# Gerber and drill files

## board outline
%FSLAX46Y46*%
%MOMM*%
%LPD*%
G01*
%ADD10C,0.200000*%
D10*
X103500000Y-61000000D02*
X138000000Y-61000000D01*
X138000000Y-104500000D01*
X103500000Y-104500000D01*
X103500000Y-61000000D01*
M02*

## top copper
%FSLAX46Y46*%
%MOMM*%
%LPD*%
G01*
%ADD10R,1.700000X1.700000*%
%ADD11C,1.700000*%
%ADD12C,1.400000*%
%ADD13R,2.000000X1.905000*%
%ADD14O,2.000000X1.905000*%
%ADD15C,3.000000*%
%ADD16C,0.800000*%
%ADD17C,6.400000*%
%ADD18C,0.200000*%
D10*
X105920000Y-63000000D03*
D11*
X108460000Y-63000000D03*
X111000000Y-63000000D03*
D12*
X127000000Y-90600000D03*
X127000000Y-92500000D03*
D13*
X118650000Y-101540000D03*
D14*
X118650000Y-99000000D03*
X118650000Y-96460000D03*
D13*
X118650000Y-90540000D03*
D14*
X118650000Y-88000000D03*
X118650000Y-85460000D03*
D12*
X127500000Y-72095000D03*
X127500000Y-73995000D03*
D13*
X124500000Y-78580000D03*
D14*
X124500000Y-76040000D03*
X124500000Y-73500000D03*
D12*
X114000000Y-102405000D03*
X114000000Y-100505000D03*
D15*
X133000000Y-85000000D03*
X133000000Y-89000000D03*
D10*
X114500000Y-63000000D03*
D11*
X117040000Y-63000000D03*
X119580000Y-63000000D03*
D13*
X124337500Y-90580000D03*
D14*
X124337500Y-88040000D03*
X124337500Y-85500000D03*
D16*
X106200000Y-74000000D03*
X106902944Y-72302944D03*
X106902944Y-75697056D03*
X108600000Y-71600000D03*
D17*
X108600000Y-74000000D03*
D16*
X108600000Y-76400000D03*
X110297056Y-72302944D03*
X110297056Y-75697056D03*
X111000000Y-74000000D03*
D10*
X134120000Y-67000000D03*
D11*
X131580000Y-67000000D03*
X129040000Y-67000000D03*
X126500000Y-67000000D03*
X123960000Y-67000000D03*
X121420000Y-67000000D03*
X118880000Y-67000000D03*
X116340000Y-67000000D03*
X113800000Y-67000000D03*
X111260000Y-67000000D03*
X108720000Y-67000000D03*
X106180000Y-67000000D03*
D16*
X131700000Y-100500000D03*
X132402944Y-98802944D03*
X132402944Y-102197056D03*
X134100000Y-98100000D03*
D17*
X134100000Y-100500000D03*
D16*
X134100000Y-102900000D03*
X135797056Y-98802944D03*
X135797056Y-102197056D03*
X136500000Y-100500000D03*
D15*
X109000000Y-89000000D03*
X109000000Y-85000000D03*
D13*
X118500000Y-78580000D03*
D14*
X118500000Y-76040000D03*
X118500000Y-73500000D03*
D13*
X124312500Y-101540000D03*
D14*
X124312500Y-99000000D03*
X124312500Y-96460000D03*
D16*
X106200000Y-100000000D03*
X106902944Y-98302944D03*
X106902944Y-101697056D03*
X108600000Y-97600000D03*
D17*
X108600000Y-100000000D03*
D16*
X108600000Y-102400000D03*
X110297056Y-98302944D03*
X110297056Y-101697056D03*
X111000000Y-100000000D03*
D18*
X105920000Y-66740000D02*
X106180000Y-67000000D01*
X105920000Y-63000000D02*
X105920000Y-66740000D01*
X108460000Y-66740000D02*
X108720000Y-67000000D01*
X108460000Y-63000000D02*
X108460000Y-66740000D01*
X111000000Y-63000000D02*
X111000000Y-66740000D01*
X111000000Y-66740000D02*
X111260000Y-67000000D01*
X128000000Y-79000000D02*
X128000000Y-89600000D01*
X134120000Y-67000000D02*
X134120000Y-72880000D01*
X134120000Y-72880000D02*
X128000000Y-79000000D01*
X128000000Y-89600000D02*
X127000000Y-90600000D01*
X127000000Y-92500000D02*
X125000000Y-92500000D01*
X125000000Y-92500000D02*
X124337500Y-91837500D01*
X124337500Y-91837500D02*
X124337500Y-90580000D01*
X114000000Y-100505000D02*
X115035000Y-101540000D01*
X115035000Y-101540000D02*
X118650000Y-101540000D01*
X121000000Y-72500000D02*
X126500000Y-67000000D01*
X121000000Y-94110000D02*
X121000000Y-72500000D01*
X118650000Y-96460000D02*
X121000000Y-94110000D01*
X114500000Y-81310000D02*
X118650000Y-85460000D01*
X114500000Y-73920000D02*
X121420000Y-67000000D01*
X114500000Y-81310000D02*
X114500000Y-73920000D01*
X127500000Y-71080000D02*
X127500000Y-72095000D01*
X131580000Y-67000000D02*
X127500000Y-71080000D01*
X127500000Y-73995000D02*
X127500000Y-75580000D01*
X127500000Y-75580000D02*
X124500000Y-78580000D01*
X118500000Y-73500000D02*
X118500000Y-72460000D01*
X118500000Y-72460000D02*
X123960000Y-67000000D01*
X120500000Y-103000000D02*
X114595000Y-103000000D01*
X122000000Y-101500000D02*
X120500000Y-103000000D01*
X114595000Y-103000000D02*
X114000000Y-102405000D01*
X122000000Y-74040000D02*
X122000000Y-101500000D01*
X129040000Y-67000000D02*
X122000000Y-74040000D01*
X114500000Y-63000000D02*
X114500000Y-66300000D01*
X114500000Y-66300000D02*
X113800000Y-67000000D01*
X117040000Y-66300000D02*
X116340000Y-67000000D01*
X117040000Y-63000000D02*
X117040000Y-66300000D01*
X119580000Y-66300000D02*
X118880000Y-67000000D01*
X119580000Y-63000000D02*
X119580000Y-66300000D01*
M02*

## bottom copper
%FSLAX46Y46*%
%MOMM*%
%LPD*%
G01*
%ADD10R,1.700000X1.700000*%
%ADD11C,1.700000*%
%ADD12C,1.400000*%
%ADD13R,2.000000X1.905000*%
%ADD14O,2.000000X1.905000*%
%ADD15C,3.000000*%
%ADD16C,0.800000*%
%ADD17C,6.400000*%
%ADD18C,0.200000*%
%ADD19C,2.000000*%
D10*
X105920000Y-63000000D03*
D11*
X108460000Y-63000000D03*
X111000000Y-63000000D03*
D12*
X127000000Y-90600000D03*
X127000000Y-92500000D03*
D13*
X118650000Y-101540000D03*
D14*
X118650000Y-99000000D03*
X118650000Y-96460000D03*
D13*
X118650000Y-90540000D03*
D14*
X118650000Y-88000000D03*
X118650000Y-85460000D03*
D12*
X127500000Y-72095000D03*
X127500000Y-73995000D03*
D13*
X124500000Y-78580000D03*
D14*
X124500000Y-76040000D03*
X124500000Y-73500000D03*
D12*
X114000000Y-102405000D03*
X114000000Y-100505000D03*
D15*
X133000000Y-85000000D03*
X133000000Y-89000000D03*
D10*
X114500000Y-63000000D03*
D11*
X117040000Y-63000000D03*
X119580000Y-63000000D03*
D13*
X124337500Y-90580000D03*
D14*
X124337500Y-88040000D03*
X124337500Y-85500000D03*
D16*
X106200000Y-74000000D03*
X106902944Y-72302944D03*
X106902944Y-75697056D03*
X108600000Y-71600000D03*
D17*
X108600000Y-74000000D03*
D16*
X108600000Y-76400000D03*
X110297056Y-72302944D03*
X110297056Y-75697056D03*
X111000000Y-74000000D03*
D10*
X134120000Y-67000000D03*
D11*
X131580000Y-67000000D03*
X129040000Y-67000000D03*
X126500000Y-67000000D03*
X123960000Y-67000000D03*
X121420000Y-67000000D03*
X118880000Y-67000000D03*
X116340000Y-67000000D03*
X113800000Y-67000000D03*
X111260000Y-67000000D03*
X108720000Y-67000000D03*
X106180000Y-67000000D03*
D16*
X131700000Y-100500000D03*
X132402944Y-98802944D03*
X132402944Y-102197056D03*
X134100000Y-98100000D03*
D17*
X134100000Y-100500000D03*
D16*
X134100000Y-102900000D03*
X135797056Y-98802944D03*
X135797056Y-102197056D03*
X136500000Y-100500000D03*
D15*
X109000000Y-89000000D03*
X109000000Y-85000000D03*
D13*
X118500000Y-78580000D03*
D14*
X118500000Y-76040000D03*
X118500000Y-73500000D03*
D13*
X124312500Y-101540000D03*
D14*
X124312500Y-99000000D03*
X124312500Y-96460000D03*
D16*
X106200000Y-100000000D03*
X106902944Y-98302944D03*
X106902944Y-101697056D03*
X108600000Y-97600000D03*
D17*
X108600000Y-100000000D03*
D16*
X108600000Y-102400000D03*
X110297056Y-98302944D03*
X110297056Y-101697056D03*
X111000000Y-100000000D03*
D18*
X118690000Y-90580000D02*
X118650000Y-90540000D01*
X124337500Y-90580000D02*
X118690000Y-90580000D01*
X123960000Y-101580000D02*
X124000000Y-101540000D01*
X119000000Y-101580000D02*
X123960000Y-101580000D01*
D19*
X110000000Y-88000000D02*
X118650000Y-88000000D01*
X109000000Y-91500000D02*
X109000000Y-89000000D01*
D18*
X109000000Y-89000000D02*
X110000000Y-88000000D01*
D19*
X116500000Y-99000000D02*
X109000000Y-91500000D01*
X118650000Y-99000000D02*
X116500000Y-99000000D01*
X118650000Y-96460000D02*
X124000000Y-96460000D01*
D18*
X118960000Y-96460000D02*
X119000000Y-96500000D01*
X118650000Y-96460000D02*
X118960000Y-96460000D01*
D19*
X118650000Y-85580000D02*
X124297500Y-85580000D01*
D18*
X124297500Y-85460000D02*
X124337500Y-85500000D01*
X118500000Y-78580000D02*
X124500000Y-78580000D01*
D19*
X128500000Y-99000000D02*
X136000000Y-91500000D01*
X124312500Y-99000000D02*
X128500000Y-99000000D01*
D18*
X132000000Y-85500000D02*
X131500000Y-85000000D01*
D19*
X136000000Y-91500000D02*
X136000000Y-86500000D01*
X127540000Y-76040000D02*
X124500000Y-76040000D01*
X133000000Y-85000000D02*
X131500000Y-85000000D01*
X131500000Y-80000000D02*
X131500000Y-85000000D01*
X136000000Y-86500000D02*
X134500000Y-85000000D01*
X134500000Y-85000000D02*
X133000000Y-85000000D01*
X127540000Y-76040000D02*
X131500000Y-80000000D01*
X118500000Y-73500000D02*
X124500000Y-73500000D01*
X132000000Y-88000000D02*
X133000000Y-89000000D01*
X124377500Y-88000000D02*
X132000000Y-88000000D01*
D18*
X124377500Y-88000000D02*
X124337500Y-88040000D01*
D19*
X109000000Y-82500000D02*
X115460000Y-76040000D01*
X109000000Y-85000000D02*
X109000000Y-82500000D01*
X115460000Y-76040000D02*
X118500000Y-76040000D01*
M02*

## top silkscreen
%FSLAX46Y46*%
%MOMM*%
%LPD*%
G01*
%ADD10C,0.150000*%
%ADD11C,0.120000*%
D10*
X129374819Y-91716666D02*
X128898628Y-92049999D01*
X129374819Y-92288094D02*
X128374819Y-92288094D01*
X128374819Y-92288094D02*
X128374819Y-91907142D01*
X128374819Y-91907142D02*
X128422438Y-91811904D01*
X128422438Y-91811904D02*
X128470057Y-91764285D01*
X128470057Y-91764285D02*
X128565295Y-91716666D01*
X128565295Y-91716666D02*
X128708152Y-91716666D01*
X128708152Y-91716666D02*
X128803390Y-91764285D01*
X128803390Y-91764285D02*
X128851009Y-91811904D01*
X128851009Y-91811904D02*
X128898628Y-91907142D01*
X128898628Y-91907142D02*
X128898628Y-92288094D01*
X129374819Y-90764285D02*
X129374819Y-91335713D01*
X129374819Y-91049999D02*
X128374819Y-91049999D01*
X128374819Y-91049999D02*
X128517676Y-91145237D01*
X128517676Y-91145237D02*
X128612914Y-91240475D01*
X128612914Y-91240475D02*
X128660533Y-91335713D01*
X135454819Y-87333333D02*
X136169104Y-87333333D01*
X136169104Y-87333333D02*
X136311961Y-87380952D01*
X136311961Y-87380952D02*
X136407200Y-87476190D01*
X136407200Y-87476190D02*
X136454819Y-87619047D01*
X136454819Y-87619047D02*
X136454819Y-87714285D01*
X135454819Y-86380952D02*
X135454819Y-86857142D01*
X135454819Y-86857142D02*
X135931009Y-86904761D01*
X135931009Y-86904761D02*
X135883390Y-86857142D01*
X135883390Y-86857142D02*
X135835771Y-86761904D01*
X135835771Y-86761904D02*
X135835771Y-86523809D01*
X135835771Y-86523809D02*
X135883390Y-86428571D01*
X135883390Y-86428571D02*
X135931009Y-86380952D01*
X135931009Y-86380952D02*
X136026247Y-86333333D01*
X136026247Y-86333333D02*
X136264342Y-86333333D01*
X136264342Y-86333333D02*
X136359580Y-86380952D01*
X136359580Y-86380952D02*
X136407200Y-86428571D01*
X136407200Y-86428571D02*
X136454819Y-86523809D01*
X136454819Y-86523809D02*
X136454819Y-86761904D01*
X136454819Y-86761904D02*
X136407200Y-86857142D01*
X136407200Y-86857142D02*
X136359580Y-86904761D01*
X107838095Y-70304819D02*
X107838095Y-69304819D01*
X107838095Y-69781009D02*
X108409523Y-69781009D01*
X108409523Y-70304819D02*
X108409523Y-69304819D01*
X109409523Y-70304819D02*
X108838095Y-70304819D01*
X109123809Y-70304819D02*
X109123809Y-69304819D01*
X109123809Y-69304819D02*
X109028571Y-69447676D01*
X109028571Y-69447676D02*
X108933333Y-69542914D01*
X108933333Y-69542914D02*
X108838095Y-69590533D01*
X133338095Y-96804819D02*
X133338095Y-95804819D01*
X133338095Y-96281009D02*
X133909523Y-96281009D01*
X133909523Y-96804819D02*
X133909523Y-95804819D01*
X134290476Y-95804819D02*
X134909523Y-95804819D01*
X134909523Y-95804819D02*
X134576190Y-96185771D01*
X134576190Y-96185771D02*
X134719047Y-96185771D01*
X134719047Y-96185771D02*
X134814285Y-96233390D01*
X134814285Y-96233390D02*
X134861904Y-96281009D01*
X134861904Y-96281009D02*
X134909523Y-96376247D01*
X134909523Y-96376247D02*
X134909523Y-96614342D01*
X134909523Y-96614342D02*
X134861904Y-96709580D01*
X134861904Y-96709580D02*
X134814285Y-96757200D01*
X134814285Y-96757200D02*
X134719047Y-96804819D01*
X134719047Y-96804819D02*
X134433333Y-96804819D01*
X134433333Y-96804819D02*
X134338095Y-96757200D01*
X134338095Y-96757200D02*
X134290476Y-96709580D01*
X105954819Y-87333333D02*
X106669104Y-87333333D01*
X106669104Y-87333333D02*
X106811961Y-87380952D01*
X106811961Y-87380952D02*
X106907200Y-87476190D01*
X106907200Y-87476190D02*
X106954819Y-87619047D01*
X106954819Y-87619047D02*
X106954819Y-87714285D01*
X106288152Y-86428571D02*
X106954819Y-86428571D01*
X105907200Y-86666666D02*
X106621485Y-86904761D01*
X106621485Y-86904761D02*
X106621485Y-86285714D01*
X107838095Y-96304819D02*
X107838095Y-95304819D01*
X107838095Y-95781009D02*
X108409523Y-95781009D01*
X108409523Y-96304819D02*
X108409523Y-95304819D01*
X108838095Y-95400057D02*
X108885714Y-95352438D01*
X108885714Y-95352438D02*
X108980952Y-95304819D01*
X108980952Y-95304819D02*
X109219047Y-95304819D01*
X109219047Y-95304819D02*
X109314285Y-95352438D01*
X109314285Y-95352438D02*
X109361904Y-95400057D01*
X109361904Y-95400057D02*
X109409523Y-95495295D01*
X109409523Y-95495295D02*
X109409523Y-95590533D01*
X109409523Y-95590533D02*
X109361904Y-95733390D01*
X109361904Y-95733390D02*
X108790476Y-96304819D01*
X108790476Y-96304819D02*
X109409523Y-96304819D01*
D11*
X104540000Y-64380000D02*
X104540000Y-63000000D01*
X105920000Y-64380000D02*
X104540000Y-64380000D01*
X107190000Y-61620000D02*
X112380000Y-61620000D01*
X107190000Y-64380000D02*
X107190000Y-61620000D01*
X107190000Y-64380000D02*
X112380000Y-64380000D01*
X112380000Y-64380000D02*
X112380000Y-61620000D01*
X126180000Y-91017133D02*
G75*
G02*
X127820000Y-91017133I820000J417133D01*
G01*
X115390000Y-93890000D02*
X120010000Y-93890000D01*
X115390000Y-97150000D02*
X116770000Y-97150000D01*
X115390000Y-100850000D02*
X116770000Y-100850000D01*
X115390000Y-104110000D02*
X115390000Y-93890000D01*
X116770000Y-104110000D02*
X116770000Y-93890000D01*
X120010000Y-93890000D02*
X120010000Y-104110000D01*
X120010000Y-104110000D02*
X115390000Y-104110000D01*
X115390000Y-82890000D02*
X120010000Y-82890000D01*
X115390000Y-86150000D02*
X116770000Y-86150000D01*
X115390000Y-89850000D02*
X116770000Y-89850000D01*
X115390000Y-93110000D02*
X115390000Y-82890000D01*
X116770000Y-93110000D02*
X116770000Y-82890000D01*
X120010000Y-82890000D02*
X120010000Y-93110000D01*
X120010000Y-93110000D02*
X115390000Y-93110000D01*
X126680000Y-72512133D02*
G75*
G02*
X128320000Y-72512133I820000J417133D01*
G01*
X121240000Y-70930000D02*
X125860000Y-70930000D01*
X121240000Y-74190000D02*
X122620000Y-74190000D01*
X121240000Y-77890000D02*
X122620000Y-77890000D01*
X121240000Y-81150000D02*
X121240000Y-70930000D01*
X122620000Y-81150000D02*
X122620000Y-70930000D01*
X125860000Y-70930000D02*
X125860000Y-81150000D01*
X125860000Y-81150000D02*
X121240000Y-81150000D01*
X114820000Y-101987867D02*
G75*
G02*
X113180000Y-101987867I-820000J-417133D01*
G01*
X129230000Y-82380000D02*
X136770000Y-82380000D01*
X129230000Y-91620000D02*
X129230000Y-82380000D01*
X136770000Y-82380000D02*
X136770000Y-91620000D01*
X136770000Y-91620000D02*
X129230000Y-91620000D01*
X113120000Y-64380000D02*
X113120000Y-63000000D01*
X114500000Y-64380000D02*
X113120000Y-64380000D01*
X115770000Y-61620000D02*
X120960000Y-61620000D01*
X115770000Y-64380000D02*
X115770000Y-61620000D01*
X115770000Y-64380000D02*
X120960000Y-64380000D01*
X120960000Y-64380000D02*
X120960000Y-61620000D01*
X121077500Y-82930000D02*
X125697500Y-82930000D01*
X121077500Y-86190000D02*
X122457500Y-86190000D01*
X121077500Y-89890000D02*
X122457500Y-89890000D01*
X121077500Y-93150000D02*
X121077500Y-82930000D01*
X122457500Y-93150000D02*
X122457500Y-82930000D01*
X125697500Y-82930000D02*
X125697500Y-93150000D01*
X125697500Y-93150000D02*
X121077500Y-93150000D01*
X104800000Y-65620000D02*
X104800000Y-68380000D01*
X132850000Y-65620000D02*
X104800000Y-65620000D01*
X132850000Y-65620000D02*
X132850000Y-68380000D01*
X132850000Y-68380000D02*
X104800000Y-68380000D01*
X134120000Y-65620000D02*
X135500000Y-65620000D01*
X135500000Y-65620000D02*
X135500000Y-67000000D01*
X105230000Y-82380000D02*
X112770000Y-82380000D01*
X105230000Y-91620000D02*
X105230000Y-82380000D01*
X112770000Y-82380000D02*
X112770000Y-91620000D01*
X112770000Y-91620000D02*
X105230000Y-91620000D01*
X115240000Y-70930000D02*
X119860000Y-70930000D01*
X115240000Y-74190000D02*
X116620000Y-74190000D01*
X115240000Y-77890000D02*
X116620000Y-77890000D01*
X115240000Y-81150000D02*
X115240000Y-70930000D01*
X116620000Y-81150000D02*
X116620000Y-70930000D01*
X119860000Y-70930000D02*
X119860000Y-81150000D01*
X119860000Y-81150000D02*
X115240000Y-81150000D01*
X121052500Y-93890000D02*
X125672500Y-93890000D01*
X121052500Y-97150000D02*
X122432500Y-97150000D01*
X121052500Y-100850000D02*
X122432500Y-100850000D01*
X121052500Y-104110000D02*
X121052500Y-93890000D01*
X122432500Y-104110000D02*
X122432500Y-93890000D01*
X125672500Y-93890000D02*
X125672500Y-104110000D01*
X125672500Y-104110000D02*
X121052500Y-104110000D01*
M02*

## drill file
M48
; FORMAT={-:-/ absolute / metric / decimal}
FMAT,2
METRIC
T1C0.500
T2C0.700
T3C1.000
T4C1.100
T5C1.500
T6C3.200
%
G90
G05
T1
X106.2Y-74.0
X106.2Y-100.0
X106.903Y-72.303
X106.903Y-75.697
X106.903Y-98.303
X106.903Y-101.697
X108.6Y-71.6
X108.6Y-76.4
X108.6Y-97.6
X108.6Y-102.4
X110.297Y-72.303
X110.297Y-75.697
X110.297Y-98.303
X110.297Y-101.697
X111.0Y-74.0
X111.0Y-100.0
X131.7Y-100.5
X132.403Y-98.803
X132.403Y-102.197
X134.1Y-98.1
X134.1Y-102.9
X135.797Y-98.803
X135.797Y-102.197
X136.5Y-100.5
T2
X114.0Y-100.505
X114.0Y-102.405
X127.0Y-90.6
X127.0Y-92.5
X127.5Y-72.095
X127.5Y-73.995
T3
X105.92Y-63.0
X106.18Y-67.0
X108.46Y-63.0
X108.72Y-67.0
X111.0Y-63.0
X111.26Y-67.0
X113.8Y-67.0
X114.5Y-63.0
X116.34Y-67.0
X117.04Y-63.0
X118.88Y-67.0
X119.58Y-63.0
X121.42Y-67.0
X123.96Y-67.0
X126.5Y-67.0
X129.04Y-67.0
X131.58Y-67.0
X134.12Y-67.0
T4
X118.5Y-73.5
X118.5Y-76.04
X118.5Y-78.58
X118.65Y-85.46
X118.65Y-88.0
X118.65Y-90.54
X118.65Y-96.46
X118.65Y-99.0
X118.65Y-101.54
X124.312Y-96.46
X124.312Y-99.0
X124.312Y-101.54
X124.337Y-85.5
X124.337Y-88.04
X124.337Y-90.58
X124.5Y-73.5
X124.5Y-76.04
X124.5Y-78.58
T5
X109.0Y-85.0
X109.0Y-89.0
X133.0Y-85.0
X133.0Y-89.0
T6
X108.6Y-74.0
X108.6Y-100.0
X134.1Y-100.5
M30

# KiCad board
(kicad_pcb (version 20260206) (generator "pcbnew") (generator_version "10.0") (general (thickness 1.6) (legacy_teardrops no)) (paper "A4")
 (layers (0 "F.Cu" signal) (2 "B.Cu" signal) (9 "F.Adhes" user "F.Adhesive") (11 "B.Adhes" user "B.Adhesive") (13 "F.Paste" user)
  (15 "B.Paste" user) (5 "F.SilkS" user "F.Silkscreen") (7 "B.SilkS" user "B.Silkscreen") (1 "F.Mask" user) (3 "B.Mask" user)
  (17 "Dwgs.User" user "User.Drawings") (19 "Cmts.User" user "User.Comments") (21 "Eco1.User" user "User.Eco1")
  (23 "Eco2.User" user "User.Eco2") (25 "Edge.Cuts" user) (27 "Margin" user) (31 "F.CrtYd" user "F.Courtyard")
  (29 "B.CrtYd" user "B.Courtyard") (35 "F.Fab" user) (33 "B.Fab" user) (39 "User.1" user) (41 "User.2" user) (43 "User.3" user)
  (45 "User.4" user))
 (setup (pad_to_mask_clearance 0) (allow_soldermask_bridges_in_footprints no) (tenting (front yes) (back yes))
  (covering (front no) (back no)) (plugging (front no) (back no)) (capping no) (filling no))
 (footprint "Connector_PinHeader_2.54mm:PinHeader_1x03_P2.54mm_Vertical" (layer "F.Cu") (at 105.92 63 90)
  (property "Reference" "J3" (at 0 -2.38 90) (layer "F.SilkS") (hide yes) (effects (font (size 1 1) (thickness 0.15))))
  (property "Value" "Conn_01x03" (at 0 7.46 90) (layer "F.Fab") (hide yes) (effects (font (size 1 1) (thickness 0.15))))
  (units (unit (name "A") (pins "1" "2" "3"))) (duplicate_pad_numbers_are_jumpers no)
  (fp_line (start -1.38 -1.38) (end 0 -1.38) (stroke (width 0.12) (type solid)) (layer "F.SilkS"))
  (fp_line (start -1.38 0) (end -1.38 -1.38) (stroke (width 0.12) (type solid)) (layer "F.SilkS"))
  (fp_line (start 1.38 1.27) (end 1.38 6.46) (stroke (width 0.12) (type solid)) (layer "F.SilkS"))
  (fp_line (start -1.38 1.27) (end 1.38 1.27) (stroke (width 0.12) (type solid)) (layer "F.SilkS"))
  (fp_line (start -1.38 1.27) (end -1.38 6.46) (stroke (width 0.12) (type solid)) (layer "F.SilkS"))
  (fp_line (start -1.38 6.46) (end 1.38 6.46) (stroke (width 0.12) (type solid)) (layer "F.SilkS"))
  (pad "1" thru_hole rect (at 0 0 90) (size 1.7 1.7) (drill 1) (layers "*.Cu" "*.Mask") (remove_unused_layers no) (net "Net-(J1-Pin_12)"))
  (pad "2" thru_hole circle (at 0 2.54 90) (size 1.7 1.7) (drill 1) (layers "*.Cu" "*.Mask") (remove_unused_layers no)
   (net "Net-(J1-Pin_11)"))
  (pad "3" thru_hole circle (at 0 5.08 90) (size 1.7 1.7) (drill 1) (layers "*.Cu" "*.Mask") (remove_unused_layers no)
   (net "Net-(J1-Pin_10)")))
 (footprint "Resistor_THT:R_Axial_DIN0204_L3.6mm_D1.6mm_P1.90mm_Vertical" (layer "F.Cu") (at 127 90.6 -90)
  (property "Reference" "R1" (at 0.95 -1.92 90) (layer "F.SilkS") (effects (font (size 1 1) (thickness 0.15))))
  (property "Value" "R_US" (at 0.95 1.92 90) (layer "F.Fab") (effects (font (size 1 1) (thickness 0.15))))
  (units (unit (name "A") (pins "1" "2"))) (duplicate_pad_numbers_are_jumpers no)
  (fp_arc (start 0.417133 0.82) (mid -0.92 0) (end 0.417133 -0.82) (stroke (width 0.12) (type solid)) (layer "F.SilkS"))
  (pad "1" thru_hole circle (at 0 0 270) (size 1.4 1.4) (drill 0.7) (layers "*.Cu" "*.Mask") (remove_unused_layers no)
   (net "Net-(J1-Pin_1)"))
  (pad "2" thru_hole circle (at 1.9 0 270) (size 1.4 1.4) (drill 0.7) (layers "*.Cu" "*.Mask") (remove_unused_layers no) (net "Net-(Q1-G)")))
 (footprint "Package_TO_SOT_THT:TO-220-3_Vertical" (layer "F.Cu") (at 118.65 101.54 90)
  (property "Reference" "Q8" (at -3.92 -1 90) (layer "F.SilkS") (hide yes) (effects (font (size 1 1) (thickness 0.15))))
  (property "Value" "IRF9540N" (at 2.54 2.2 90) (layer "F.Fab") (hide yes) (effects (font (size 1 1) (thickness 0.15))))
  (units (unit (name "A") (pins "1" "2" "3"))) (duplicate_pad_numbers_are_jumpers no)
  (fp_line (start 7.65 -3.26) (end 7.65 1.36) (stroke (width 0.12) (type solid)) (layer "F.SilkS"))
  (fp_line (start 4.39 -3.26) (end 4.39 -1.88) (stroke (width 0.12) (type solid)) (layer "F.SilkS"))
  (fp_line (start 0.69 -3.26) (end 0.69 -1.88) (stroke (width 0.12) (type solid)) (layer "F.SilkS"))
  (fp_line (start -2.57 -3.26) (end 7.65 -3.26) (stroke (width 0.12) (type solid)) (layer "F.SilkS"))
  (fp_line (start -2.57 -1.88) (end 7.65 -1.88) (stroke (width 0.12) (type solid)) (layer "F.SilkS"))
  (fp_line (start 7.65 1.36) (end -2.57 1.36) (stroke (width 0.12) (type solid)) (layer "F.SilkS"))
  (fp_line (start -2.57 1.36) (end -2.57 -3.26) (stroke (width 0.12) (type solid)) (layer "F.SilkS"))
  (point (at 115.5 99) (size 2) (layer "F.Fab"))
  (pad "1" thru_hole rect (at 0 0 90) (size 1.905 2) (drill 1.1) (layers "*.Cu" "*.Mask") (remove_unused_layers no) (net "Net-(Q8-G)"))
  (pad "2" thru_hole oval (at 2.54 0 90) (size 1.905 2) (drill 1.1) (layers "*.Cu" "*.Mask") (remove_unused_layers no) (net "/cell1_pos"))
  (pad "3" thru_hole oval (at 5.08 0 90) (size 1.905 2) (drill 1.1) (layers "*.Cu" "*.Mask") (remove_unused_layers no) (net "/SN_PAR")))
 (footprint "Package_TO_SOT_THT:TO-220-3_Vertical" (layer "F.Cu") (at 118.65 90.54 90)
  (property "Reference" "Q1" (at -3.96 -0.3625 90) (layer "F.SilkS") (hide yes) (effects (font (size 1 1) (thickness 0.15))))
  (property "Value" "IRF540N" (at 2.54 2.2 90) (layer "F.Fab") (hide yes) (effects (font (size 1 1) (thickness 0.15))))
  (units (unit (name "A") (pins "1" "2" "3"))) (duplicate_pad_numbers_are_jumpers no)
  (fp_line (start 7.65 -3.26) (end 7.65 1.36) (stroke (width 0.12) (type solid)) (layer "F.SilkS"))
  (fp_line (start 4.39 -3.26) (end 4.39 -1.88) (stroke (width 0.12) (type solid)) (layer "F.SilkS"))
  (fp_line (start 0.69 -3.26) (end 0.69 -1.88) (stroke (width 0.12) (type solid)) (layer "F.SilkS"))
  (fp_line (start -2.57 -3.26) (end 7.65 -3.26) (stroke (width 0.12) (type solid)) (layer "F.SilkS"))
  (fp_line (start -2.57 -1.88) (end 7.65 -1.88) (stroke (width 0.12) (type solid)) (layer "F.SilkS"))
  (fp_line (start 7.65 1.36) (end -2.57 1.36) (stroke (width 0.12) (type solid)) (layer "F.SilkS"))
  (fp_line (start -2.57 1.36) (end -2.57 -3.26) (stroke (width 0.12) (type solid)) (layer "F.SilkS"))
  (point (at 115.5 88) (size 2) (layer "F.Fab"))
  (pad "1" thru_hole rect (at 0 0 90) (size 1.905 2) (drill 1.1) (layers "*.Cu" "*.Mask") (remove_unused_layers no) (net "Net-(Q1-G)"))
  (pad "2" thru_hole oval (at 2.54 0 90) (size 1.905 2) (drill 1.1) (layers "*.Cu" "*.Mask") (remove_unused_layers no) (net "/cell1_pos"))
  (pad "3" thru_hole oval (at 5.08 0 90) (size 1.905 2) (drill 1.1) (layers "*.Cu" "*.Mask") (remove_unused_layers no) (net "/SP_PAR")))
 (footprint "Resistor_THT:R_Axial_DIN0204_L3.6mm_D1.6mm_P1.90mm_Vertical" (layer "F.Cu") (at 127.5 72.095 -90)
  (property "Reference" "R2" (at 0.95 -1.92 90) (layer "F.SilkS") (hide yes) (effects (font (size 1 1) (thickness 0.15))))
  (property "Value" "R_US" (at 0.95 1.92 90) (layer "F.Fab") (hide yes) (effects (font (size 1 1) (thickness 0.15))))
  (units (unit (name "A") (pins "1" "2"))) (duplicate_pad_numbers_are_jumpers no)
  (fp_arc (start 0.417133 0.82) (mid -0.92 0) (end 0.417133 -0.82) (stroke (width 0.12) (type solid)) (layer "F.SilkS"))
  (pad "1" thru_hole circle (at 0 0 270) (size 1.4 1.4) (drill 0.7) (layers "*.Cu" "*.Mask") (remove_unused_layers no)
   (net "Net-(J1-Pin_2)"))
  (pad "2" thru_hole circle (at 1.9 0 270) (size 1.4 1.4) (drill 0.7) (layers "*.Cu" "*.Mask") (remove_unused_layers no) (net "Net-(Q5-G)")))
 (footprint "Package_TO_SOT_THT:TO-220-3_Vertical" (layer "F.Cu") (at 124.5 78.58 90)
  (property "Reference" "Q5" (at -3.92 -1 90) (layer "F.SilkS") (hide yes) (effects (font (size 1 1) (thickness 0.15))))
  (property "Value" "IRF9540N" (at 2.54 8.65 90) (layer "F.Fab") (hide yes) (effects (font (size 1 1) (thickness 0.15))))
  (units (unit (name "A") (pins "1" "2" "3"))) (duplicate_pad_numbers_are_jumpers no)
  (fp_line (start 7.65 -3.26) (end 7.65 1.36) (stroke (width 0.12) (type solid)) (layer "F.SilkS"))
  (fp_line (start 4.39 -3.26) (end 4.39 -1.88) (stroke (width 0.12) (type solid)) (layer "F.SilkS"))
  (fp_line (start 0.69 -3.26) (end 0.69 -1.88) (stroke (width 0.12) (type solid)) (layer "F.SilkS"))
  (fp_line (start -2.57 -3.26) (end 7.65 -3.26) (stroke (width 0.12) (type solid)) (layer "F.SilkS"))
  (fp_line (start -2.57 -1.88) (end 7.65 -1.88) (stroke (width 0.12) (type solid)) (layer "F.SilkS"))
  (fp_line (start 7.65 1.36) (end -2.57 1.36) (stroke (width 0.12) (type solid)) (layer "F.SilkS"))
  (fp_line (start -2.57 1.36) (end -2.57 -3.26) (stroke (width 0.12) (type solid)) (layer "F.SilkS"))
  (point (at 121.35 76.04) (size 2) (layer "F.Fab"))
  (pad "1" thru_hole rect (at 0 0 90) (size 1.905 2) (drill 1.1) (layers "*.Cu" "*.Mask") (remove_unused_layers no) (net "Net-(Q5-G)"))
  (pad "2" thru_hole oval (at 2.54 0 90) (size 1.905 2) (drill 1.1) (layers "*.Cu" "*.Mask") (remove_unused_layers no) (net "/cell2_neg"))
  (pad "3" thru_hole oval (at 5.08 0 90) (size 1.905 2) (drill 1.1) (layers "*.Cu" "*.Mask") (remove_unused_layers no) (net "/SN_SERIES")))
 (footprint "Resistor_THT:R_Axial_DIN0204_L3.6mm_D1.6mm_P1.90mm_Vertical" (layer "F.Cu") (at 114 102.405 90)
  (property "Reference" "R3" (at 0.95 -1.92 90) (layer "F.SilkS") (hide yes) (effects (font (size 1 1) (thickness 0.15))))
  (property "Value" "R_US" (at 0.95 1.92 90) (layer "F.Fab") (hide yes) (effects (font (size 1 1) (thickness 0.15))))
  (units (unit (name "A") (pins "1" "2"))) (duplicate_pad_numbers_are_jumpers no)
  (fp_arc (start 0.417133 0.82) (mid -0.92 0) (end 0.417133 -0.82) (stroke (width 0.12) (type solid)) (layer "F.SilkS"))
  (pad "1" thru_hole circle (at 0 0 90) (size 1.4 1.4) (drill 0.7) (layers "*.Cu" "*.Mask") (remove_unused_layers no) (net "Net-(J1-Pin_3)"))
  (pad "2" thru_hole circle (at 1.9 0 90) (size 1.4 1.4) (drill 0.7) (layers "*.Cu" "*.Mask") (remove_unused_layers no) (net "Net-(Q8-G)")))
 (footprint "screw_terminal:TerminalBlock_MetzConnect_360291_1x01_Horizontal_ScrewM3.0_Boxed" (layer "F.Cu") (at 133 85 -90)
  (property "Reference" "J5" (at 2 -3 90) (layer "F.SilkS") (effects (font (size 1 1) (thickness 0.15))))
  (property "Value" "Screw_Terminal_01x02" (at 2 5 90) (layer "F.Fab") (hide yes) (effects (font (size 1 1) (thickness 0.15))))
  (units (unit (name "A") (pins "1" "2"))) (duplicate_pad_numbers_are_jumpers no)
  (fp_line (start -2.62 3.77) (end -2.62 -3.77) (stroke (width 0.12) (type solid)) (layer "F.SilkS"))
  (fp_line (start 6.62 3.77) (end -2.62 3.77) (stroke (width 0.12) (type solid)) (layer "F.SilkS"))
  (fp_line (start -2.62 -3.77) (end 6.62 -3.77) (stroke (width 0.12) (type solid)) (layer "F.SilkS"))
  (fp_line (start 6.62 -3.77) (end 6.62 3.77) (stroke (width 0.12) (type solid)) (layer "F.SilkS"))
  (pad "1" thru_hole circle (at 0 0 270) (size 3 3) (drill 1.5) (layers "*.Cu" "*.Mask") (remove_unused_layers no) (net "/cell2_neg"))
  (pad "2" thru_hole circle (at 4 0 270) (size 3 3) (drill 1.5) (layers "*.Cu" "*.Mask") (remove_unused_layers no) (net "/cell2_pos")))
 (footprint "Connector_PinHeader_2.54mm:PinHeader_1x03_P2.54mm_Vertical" (layer "F.Cu") (at 114.5 63 90)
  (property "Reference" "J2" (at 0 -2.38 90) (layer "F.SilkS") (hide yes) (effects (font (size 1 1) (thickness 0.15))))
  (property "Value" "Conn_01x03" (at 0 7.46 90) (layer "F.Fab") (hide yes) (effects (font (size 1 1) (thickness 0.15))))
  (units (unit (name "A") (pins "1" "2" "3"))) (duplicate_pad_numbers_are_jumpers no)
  (fp_line (start -1.38 -1.38) (end 0 -1.38) (stroke (width 0.12) (type solid)) (layer "F.SilkS"))
  (fp_line (start -1.38 0) (end -1.38 -1.38) (stroke (width 0.12) (type solid)) (layer "F.SilkS"))
  (fp_line (start 1.38 1.27) (end 1.38 6.46) (stroke (width 0.12) (type solid)) (layer "F.SilkS"))
  (fp_line (start -1.38 1.27) (end 1.38 1.27) (stroke (width 0.12) (type solid)) (layer "F.SilkS"))
  (fp_line (start -1.38 1.27) (end -1.38 6.46) (stroke (width 0.12) (type solid)) (layer "F.SilkS"))
  (fp_line (start -1.38 6.46) (end 1.38 6.46) (stroke (width 0.12) (type solid)) (layer "F.SilkS"))
  (pad "1" thru_hole rect (at 0 0 90) (size 1.7 1.7) (drill 1) (layers "*.Cu" "*.Mask") (remove_unused_layers no) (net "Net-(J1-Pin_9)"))
  (pad "2" thru_hole circle (at 0 2.54 90) (size 1.7 1.7) (drill 1) (layers "*.Cu" "*.Mask") (remove_unused_layers no)
   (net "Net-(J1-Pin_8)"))
  (pad "3" thru_hole circle (at 0 5.08 90) (size 1.7 1.7) (drill 1) (layers "*.Cu" "*.Mask") (remove_unused_layers no)
   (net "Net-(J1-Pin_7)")))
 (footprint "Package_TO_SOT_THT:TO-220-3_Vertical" (layer "F.Cu") (at 124.3375 90.58 90)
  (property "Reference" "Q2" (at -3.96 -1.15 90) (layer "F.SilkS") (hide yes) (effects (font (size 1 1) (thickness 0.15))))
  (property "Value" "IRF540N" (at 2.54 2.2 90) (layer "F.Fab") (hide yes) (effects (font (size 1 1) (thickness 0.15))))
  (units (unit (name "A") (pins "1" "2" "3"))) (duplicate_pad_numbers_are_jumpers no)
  (fp_line (start 7.65 -3.26) (end 7.65 1.36) (stroke (width 0.12) (type solid)) (layer "F.SilkS"))
  (fp_line (start 4.39 -3.26) (end 4.39 -1.88) (stroke (width 0.12) (type solid)) (layer "F.SilkS"))
  (fp_line (start 0.69 -3.26) (end 0.69 -1.88) (stroke (width 0.12) (type solid)) (layer "F.SilkS"))
  (fp_line (start -2.57 -3.26) (end 7.65 -3.26) (stroke (width 0.12) (type solid)) (layer "F.SilkS"))
  (fp_line (start -2.57 -1.88) (end 7.65 -1.88) (stroke (width 0.12) (type solid)) (layer "F.SilkS"))
  (fp_line (start 7.65 1.36) (end -2.57 1.36) (stroke (width 0.12) (type solid)) (layer "F.SilkS"))
  (fp_line (start -2.57 1.36) (end -2.57 -3.26) (stroke (width 0.12) (type solid)) (layer "F.SilkS"))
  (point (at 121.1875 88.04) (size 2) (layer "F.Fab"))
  (pad "1" thru_hole rect (at 0 0 90) (size 1.905 2) (drill 1.1) (layers "*.Cu" "*.Mask") (remove_unused_layers no) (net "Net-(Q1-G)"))
  (pad "2" thru_hole oval (at 2.54 0 90) (size 1.905 2) (drill 1.1) (layers "*.Cu" "*.Mask") (remove_unused_layers no) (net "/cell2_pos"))
  (pad "3" thru_hole oval (at 5.08 0 90) (size 1.905 2) (drill 1.1) (layers "*.Cu" "*.Mask") (remove_unused_layers no) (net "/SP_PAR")))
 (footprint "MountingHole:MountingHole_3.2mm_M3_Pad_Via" (layer "F.Cu") (at 108.6 74)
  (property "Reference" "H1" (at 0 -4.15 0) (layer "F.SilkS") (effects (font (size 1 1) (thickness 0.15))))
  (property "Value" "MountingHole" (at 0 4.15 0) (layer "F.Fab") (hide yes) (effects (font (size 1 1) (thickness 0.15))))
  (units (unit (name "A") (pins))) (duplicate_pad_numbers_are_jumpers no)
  (pad "1" thru_hole circle (at -2.4 0) (size 0.8 0.8) (drill 0.5) (layers "*.Cu" "*.Mask") (remove_unused_layers no) (zone_connect 2))
  (pad "1" thru_hole circle (at -1.697056 -1.697056) (size 0.8 0.8) (drill 0.5) (layers "*.Cu" "*.Mask") (remove_unused_layers no)
   (zone_connect 2))
  (pad "1" thru_hole circle (at -1.697056 1.697056) (size 0.8 0.8) (drill 0.5) (layers "*.Cu" "*.Mask") (remove_unused_layers no)
   (zone_connect 2))
  (pad "1" thru_hole circle (at 0 -2.4) (size 0.8 0.8) (drill 0.5) (layers "*.Cu" "*.Mask") (remove_unused_layers no) (zone_connect 2))
  (pad "1" thru_hole circle (at 0 0) (size 6.4 6.4) (drill 3.2) (layers "*.Cu" "*.Mask") (remove_unused_layers no) (zone_connect 2))
  (pad "1" thru_hole circle (at 0 2.4) (size 0.8 0.8) (drill 0.5) (layers "*.Cu" "*.Mask") (remove_unused_layers no) (zone_connect 2))
  (pad "1" thru_hole circle (at 1.697056 -1.697056) (size 0.8 0.8) (drill 0.5) (layers "*.Cu" "*.Mask") (remove_unused_layers no)
   (zone_connect 2))
  (pad "1" thru_hole circle (at 1.697056 1.697056) (size 0.8 0.8) (drill 0.5) (layers "*.Cu" "*.Mask") (remove_unused_layers no)
   (zone_connect 2))
  (pad "1" thru_hole circle (at 2.4 0) (size 0.8 0.8) (drill 0.5) (layers "*.Cu" "*.Mask") (remove_unused_layers no) (zone_connect 2)))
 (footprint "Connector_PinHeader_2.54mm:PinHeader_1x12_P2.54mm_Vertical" (layer "F.Cu") (at 134.12 67 -90)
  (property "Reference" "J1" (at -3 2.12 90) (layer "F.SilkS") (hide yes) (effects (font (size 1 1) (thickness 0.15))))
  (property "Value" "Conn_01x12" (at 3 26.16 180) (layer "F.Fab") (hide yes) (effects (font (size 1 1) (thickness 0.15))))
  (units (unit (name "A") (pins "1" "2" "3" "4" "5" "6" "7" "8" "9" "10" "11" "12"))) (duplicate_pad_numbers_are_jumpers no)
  (fp_line (start -1.38 29.32) (end 1.38 29.32) (stroke (width 0.12) (type solid)) (layer "F.SilkS"))
  (fp_line (start -1.38 1.27) (end -1.38 29.32) (stroke (width 0.12) (type solid)) (layer "F.SilkS"))
  (fp_line (start -1.38 1.27) (end 1.38 1.27) (stroke (width 0.12) (type solid)) (layer "F.SilkS"))
  (fp_line (start 1.38 1.27) (end 1.38 29.32) (stroke (width 0.12) (type solid)) (layer "F.SilkS"))
  (fp_line (start -1.38 0) (end -1.38 -1.38) (stroke (width 0.12) (type solid)) (layer "F.SilkS"))
  (fp_line (start -1.38 -1.38) (end 0 -1.38) (stroke (width 0.12) (type solid)) (layer "F.SilkS"))
  (pad "1" thru_hole rect (at 0 0 270) (size 1.7 1.7) (drill 1) (layers "*.Cu" "*.Mask") (remove_unused_layers no) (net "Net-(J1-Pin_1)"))
  (pad "2" thru_hole circle (at 0 2.54 270) (size 1.7 1.7) (drill 1) (layers "*.Cu" "*.Mask") (remove_unused_layers no)
   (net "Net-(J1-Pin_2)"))
  (pad "3" thru_hole circle (at 0 5.08 270) (size 1.7 1.7) (drill 1) (layers "*.Cu" "*.Mask") (remove_unused_layers no)
   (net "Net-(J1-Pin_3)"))
  (pad "4" thru_hole circle (at 0 7.62 270) (size 1.7 1.7) (drill 1) (layers "*.Cu" "*.Mask") (remove_unused_layers no) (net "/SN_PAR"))
  (pad "5" thru_hole circle (at 0 10.16 270) (size 1.7 1.7) (drill 1) (layers "*.Cu" "*.Mask") (remove_unused_layers no) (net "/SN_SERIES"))
  (pad "6" thru_hole circle (at 0 12.7 270) (size 1.7 1.7) (drill 1) (layers "*.Cu" "*.Mask") (remove_unused_layers no) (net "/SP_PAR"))
  (pad "7" thru_hole circle (at 0 15.24 270) (size 1.7 1.7) (drill 1) (layers "*.Cu" "*.Mask") (remove_unused_layers no)
   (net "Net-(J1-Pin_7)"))
  (pad "8" thru_hole circle (at 0 17.78 270) (size 1.7 1.7) (drill 1) (layers "*.Cu" "*.Mask") (remove_unused_layers no)
   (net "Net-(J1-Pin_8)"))
  (pad "9" thru_hole circle (at 0 20.32 270) (size 1.7 1.7) (drill 1) (layers "*.Cu" "*.Mask") (remove_unused_layers no)
   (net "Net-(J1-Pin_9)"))
  (pad "10" thru_hole circle (at 0 22.86 270) (size 1.7 1.7) (drill 1) (layers "*.Cu" "*.Mask") (remove_unused_layers no)
   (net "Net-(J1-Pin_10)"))
  (pad "11" thru_hole circle (at 0 25.4 270) (size 1.7 1.7) (drill 1) (layers "*.Cu" "*.Mask") (remove_unused_layers no)
   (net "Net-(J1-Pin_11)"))
  (pad "12" thru_hole circle (at 0 27.94 270) (size 1.7 1.7) (drill 1) (layers "*.Cu" "*.Mask") (remove_unused_layers no)
   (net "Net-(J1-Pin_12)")))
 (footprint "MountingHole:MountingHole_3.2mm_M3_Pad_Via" (layer "F.Cu") (at 134.1 100.5)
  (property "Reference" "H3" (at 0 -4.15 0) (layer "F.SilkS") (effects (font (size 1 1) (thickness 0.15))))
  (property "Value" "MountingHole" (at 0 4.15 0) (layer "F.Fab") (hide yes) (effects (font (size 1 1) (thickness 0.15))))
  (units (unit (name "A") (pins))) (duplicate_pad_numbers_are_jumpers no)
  (pad "1" thru_hole circle (at -2.4 0) (size 0.8 0.8) (drill 0.5) (layers "*.Cu" "*.Mask") (remove_unused_layers no) (zone_connect 2))
  (pad "1" thru_hole circle (at -1.697056 -1.697056) (size 0.8 0.8) (drill 0.5) (layers "*.Cu" "*.Mask") (remove_unused_layers no)
   (zone_connect 2))
  (pad "1" thru_hole circle (at -1.697056 1.697056) (size 0.8 0.8) (drill 0.5) (layers "*.Cu" "*.Mask") (remove_unused_layers no)
   (zone_connect 2))
  (pad "1" thru_hole circle (at 0 -2.4) (size 0.8 0.8) (drill 0.5) (layers "*.Cu" "*.Mask") (remove_unused_layers no) (zone_connect 2))
  (pad "1" thru_hole circle (at 0 0) (size 6.4 6.4) (drill 3.2) (layers "*.Cu" "*.Mask") (remove_unused_layers no) (zone_connect 2))
  (pad "1" thru_hole circle (at 0 2.4) (size 0.8 0.8) (drill 0.5) (layers "*.Cu" "*.Mask") (remove_unused_layers no) (zone_connect 2))
  (pad "1" thru_hole circle (at 1.697056 -1.697056) (size 0.8 0.8) (drill 0.5) (layers "*.Cu" "*.Mask") (remove_unused_layers no)
   (zone_connect 2))
  (pad "1" thru_hole circle (at 1.697056 1.697056) (size 0.8 0.8) (drill 0.5) (layers "*.Cu" "*.Mask") (remove_unused_layers no)
   (zone_connect 2))
  (pad "1" thru_hole circle (at 2.4 0) (size 0.8 0.8) (drill 0.5) (layers "*.Cu" "*.Mask") (remove_unused_layers no) (zone_connect 2)))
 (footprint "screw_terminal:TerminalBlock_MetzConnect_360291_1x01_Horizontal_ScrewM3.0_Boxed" (layer "F.Cu") (at 109 89 90)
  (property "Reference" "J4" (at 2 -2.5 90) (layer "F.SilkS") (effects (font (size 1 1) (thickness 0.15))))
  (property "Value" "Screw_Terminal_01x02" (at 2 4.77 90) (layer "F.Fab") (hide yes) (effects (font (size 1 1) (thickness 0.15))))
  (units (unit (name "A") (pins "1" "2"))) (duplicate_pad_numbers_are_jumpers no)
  (fp_line (start 6.62 -3.77) (end 6.62 3.77) (stroke (width 0.12) (type solid)) (layer "F.SilkS"))
  (fp_line (start -2.62 -3.77) (end 6.62 -3.77) (stroke (width 0.12) (type solid)) (layer "F.SilkS"))
  (fp_line (start 6.62 3.77) (end -2.62 3.77) (stroke (width 0.12) (type solid)) (layer "F.SilkS"))
  (fp_line (start -2.62 3.77) (end -2.62 -3.77) (stroke (width 0.12) (type solid)) (layer "F.SilkS"))
  (pad "1" thru_hole circle (at 0 0 90) (size 3 3) (drill 1.5) (layers "*.Cu" "*.Mask") (remove_unused_layers no) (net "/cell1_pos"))
  (pad "2" thru_hole circle (at 4 0 90) (size 3 3) (drill 1.5) (layers "*.Cu" "*.Mask") (remove_unused_layers no) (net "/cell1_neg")))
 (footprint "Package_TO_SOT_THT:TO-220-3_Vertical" (layer "F.Cu") (at 118.5 78.58 90)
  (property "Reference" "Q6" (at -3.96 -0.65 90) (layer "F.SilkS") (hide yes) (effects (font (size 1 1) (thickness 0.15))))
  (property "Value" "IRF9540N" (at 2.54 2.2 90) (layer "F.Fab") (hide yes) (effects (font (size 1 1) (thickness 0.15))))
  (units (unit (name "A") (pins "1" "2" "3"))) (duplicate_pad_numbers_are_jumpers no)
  (fp_line (start 7.65 -3.26) (end 7.65 1.36) (stroke (width 0.12) (type solid)) (layer "F.SilkS"))
  (fp_line (start 4.39 -3.26) (end 4.39 -1.88) (stroke (width 0.12) (type solid)) (layer "F.SilkS"))
  (fp_line (start 0.69 -3.26) (end 0.69 -1.88) (stroke (width 0.12) (type solid)) (layer "F.SilkS"))
  (fp_line (start -2.57 -3.26) (end 7.65 -3.26) (stroke (width 0.12) (type solid)) (layer "F.SilkS"))
  (fp_line (start -2.57 -1.88) (end 7.65 -1.88) (stroke (width 0.12) (type solid)) (layer "F.SilkS"))
  (fp_line (start 7.65 1.36) (end -2.57 1.36) (stroke (width 0.12) (type solid)) (layer "F.SilkS"))
  (fp_line (start -2.57 1.36) (end -2.57 -3.26) (stroke (width 0.12) (type solid)) (layer "F.SilkS"))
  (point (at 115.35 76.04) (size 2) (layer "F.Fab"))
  (pad "1" thru_hole rect (at 0 0 90) (size 1.905 2) (drill 1.1) (layers "*.Cu" "*.Mask") (remove_unused_layers no) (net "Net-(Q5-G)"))
  (pad "2" thru_hole oval (at 2.54 0 90) (size 1.905 2) (drill 1.1) (layers "*.Cu" "*.Mask") (remove_unused_layers no) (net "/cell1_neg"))
  (pad "3" thru_hole oval (at 5.08 0 90) (size 1.905 2) (drill 1.1) (layers "*.Cu" "*.Mask") (remove_unused_layers no) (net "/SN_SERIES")))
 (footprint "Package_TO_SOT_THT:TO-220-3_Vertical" (layer "F.Cu") (at 124.3125 101.54 90)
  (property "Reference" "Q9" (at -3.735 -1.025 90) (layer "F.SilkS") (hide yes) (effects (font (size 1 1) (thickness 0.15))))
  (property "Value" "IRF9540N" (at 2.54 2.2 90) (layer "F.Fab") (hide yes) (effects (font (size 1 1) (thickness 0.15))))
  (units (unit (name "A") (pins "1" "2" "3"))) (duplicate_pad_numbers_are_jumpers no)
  (fp_line (start 7.65 -3.26) (end 7.65 1.36) (stroke (width 0.12) (type solid)) (layer "F.SilkS"))
  (fp_line (start 4.39 -3.26) (end 4.39 -1.88) (stroke (width 0.12) (type solid)) (layer "F.SilkS"))
  (fp_line (start 0.69 -3.26) (end 0.69 -1.88) (stroke (width 0.12) (type solid)) (layer "F.SilkS"))
  (fp_line (start -2.57 -3.26) (end 7.65 -3.26) (stroke (width 0.12) (type solid)) (layer "F.SilkS"))
  (fp_line (start -2.57 -1.88) (end 7.65 -1.88) (stroke (width 0.12) (type solid)) (layer "F.SilkS"))
  (fp_line (start 7.65 1.36) (end -2.57 1.36) (stroke (width 0.12) (type solid)) (layer "F.SilkS"))
  (fp_line (start -2.57 1.36) (end -2.57 -3.26) (stroke (width 0.12) (type solid)) (layer "F.SilkS"))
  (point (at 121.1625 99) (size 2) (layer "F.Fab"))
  (pad "1" thru_hole rect (at 0 0 90) (size 1.905 2) (drill 1.1) (layers "*.Cu" "*.Mask") (remove_unused_layers no) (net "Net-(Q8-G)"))
  (pad "2" thru_hole oval (at 2.54 0 90) (size 1.905 2) (drill 1.1) (layers "*.Cu" "*.Mask") (remove_unused_layers no) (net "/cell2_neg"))
  (pad "3" thru_hole oval (at 5.08 0 90) (size 1.905 2) (drill 1.1) (layers "*.Cu" "*.Mask") (remove_unused_layers no) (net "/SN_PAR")))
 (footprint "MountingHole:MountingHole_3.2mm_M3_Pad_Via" (layer "F.Cu") (at 108.6 100)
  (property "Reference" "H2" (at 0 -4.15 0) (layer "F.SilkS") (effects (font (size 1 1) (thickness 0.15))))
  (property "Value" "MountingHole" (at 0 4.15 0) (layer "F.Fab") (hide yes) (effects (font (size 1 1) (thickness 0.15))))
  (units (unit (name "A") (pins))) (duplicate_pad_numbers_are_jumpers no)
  (pad "1" thru_hole circle (at -2.4 0) (size 0.8 0.8) (drill 0.5) (layers "*.Cu" "*.Mask") (remove_unused_layers no) (zone_connect 2))
  (pad "1" thru_hole circle (at -1.697056 -1.697056) (size 0.8 0.8) (drill 0.5) (layers "*.Cu" "*.Mask") (remove_unused_layers no)
   (zone_connect 2))
  (pad "1" thru_hole circle (at -1.697056 1.697056) (size 0.8 0.8) (drill 0.5) (layers "*.Cu" "*.Mask") (remove_unused_layers no)
   (zone_connect 2))
  (pad "1" thru_hole circle (at 0 -2.4) (size 0.8 0.8) (drill 0.5) (layers "*.Cu" "*.Mask") (remove_unused_layers no) (zone_connect 2))
  (pad "1" thru_hole circle (at 0 0) (size 6.4 6.4) (drill 3.2) (layers "*.Cu" "*.Mask") (remove_unused_layers no) (zone_connect 2))
  (pad "1" thru_hole circle (at 0 2.4) (size 0.8 0.8) (drill 0.5) (layers "*.Cu" "*.Mask") (remove_unused_layers no) (zone_connect 2))
  (pad "1" thru_hole circle (at 1.697056 -1.697056) (size 0.8 0.8) (drill 0.5) (layers "*.Cu" "*.Mask") (remove_unused_layers no)
   (zone_connect 2))
  (pad "1" thru_hole circle (at 1.697056 1.697056) (size 0.8 0.8) (drill 0.5) (layers "*.Cu" "*.Mask") (remove_unused_layers no)
   (zone_connect 2))
  (pad "1" thru_hole circle (at 2.4 0) (size 0.8 0.8) (drill 0.5) (layers "*.Cu" "*.Mask") (remove_unused_layers no) (zone_connect 2)))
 (gr_rect (start 103.5 61) (end 138 104.5) (stroke (width 0.2) (type default)) (fill no) (layer "Edge.Cuts"))
 (segment (start 105.92 66.74) (end 106.18 67) (width 0.2) (layer "F.Cu") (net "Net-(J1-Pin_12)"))
 (segment (start 105.92 63) (end 105.92 66.74) (width 0.2) (layer "F.Cu") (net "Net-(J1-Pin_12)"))
 (segment (start 108.46 66.74) (end 108.72 67) (width 0.2) (layer "F.Cu") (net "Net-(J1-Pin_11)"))
 (segment (start 108.46 63) (end 108.46 66.74) (width 0.2) (layer "F.Cu") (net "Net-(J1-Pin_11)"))
 (segment (start 111 63) (end 111 66.74) (width 0.2) (layer "F.Cu") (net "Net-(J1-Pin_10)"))
 (segment (start 111 66.74) (end 111.26 67) (width 0.2) (layer "F.Cu") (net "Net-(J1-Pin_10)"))
 (segment (start 128 79) (end 128 89.6) (width 0.2) (layer "F.Cu") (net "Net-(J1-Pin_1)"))
 (segment (start 134.12 67) (end 134.12 72.88) (width 0.2) (layer "F.Cu") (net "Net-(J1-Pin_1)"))
 (segment (start 134.12 72.88) (end 128 79) (width 0.2) (layer "F.Cu") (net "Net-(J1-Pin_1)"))
 (segment (start 128 89.6) (end 127 90.6) (width 0.2) (layer "F.Cu") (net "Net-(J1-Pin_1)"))
 (segment (start 127 92.5) (end 125 92.5) (width 0.2) (layer "F.Cu") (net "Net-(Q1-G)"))
 (segment (start 125 92.5) (end 124.3375 91.8375) (width 0.2) (layer "F.Cu") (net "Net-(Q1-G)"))
 (segment (start 124.3375 91.8375) (end 124.3375 90.58) (width 0.2) (layer "F.Cu") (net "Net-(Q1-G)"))
 (segment (start 118.69 90.58) (end 118.65 90.54) (width 0.2) (layer "B.Cu") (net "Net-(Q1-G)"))
 (segment (start 124.3375 90.58) (end 118.69 90.58) (width 0.2) (layer "B.Cu") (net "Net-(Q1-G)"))
 (segment (start 114 100.505) (end 115.035 101.54) (width 0.2) (layer "F.Cu") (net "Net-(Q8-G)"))
 (segment (start 115.035 101.54) (end 118.65 101.54) (width 0.2) (layer "F.Cu") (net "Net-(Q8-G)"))
 (segment (start 123.96 101.58) (end 124 101.54) (width 0.2) (layer "B.Cu") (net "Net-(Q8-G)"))
 (segment (start 119 101.58) (end 123.96 101.58) (width 0.2) (layer "B.Cu") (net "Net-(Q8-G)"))
 (segment (start 110 88) (end 118.65 88) (width 2) (layers "B.Cu" "B.Mask") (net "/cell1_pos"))
 (segment (start 109 91.5) (end 109 89) (width 2) (layers "B.Cu" "B.Mask") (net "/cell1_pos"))
 (segment (start 109 89) (end 110 88) (width 0.2) (layer "B.Cu") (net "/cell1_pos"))
 (segment (start 116.5 99) (end 109 91.5) (width 2) (layers "B.Cu" "B.Mask") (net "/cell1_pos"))
 (segment (start 118.65 99) (end 116.5 99) (width 2) (layers "B.Cu" "B.Mask") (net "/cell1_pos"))
 (segment (start 121 72.5) (end 126.5 67) (width 0.2) (layer "F.Cu") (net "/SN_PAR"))
 (segment (start 121 94.11) (end 121 72.5) (width 0.2) (layer "F.Cu") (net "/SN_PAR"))
 (segment (start 118.65 96.46) (end 121 94.11) (width 0.2) (layer "F.Cu") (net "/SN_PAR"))
 (segment (start 118.65 96.46) (end 124 96.46) (width 2) (layers "B.Cu" "B.Mask") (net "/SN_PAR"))
 (segment (start 118.96 96.46) (end 119 96.5) (width 0.2) (layer "B.Cu") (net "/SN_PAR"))
 (segment (start 118.65 96.46) (end 118.96 96.46) (width 0.2) (layer "B.Cu") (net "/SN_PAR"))
 (segment (start 114.5 81.31) (end 118.65 85.46) (width 0.2) (layer "F.Cu") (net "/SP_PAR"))
 (segment (start 114.5 73.92) (end 121.42 67) (width 0.2) (layer "F.Cu") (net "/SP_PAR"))
 (segment (start 114.5 81.31) (end 114.5 73.92) (width 0.2) (layer "F.Cu") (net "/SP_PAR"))
 (segment (start 118.65 85.58) (end 124.2975 85.58) (width 2) (layers "B.Cu" "B.Mask") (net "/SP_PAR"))
 (segment (start 124.2975 85.46) (end 124.3375 85.5) (width 0.2) (layer "B.Cu") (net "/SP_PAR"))
 (segment (start 127.5 71.08) (end 127.5 72.095) (width 0.2) (layer "F.Cu") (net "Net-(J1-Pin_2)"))
 (segment (start 131.58 67) (end 127.5 71.08) (width 0.2) (layer "F.Cu") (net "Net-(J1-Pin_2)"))
 (segment (start 127.5 73.995) (end 127.5 75.58) (width 0.2) (layer "F.Cu") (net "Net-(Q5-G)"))
 (segment (start 127.5 75.58) (end 124.5 78.58) (width 0.2) (layer "F.Cu") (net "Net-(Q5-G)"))
 (segment (start 118.5 78.58) (end 124.5 78.58) (width 0.2) (layer "B.Cu") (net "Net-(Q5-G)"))
 (segment (start 128.5 99) (end 136 91.5) (width 2) (layers "B.Cu" "B.Mask") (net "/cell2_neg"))
 (segment (start 124.3125 99) (end 128.5 99) (width 2) (layers "B.Cu" "B.Mask") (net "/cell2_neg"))
 (segment (start 132 85.5) (end 131.5 85) (width 0.2) (layer "B.Cu") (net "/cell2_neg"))
 (segment (start 136 91.5) (end 136 86.5) (width 2) (layers "B.Cu" "B.Mask") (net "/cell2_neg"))
 (segment (start 127.54 76.04) (end 124.5 76.04) (width 2) (layers "B.Cu" "B.Mask") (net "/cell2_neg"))
 (segment (start 133 85) (end 131.5 85) (width 2) (layers "B.Cu" "B.Mask") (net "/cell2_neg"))
 (segment (start 131.5 80) (end 131.5 85) (width 2) (layers "B.Cu" "B.Mask") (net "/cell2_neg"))
 (segment (start 136 86.5) (end 134.5 85) (width 2) (layers "B.Cu" "B.Mask") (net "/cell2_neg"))
 (segment (start 134.5 85) (end 133 85) (width 2) (layers "B.Cu" "B.Mask") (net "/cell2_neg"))
 (segment (start 127.54 76.04) (end 131.5 80) (width 2) (layers "B.Cu" "B.Mask") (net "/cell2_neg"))
 (segment (start 118.5 73.5) (end 118.5 72.46) (width 0.2) (layer "F.Cu") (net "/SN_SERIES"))
 (segment (start 118.5 72.46) (end 123.96 67) (width 0.2) (layer "F.Cu") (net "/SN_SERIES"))
 (segment (start 118.5 73.5) (end 124.5 73.5) (width 2) (layers "B.Cu" "B.Mask") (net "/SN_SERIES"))
 (segment (start 120.5 103) (end 114.595 103) (width 0.2) (layer "F.Cu") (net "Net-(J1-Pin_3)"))
 (segment (start 122 101.5) (end 120.5 103) (width 0.2) (layer "F.Cu") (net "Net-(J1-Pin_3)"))
 (segment (start 114.595 103) (end 114 102.405) (width 0.2) (layer "F.Cu") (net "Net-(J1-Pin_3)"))
 (segment (start 122 74.04) (end 122 101.5) (width 0.2) (layer "F.Cu") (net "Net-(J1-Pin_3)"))
 (segment (start 129.04 67) (end 122 74.04) (width 0.2) (layer "F.Cu") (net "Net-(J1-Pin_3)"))
 (segment (start 132 88) (end 133 89) (width 2) (layer "B.Cu") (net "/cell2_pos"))
 (segment (start 124.3775 88) (end 132 88) (width 2) (layer "B.Cu") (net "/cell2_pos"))
 (segment (start 124.3775 88) (end 124.3375 88.04) (width 0.2) (layer "B.Cu") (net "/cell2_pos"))
 (segment (start 114.5 63) (end 114.5 66.3) (width 0.2) (layer "F.Cu") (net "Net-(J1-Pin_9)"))
 (segment (start 114.5 66.3) (end 113.8 67) (width 0.2) (layer "F.Cu") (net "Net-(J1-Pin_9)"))
 (segment (start 117.04 66.3) (end 116.34 67) (width 0.2) (layer "F.Cu") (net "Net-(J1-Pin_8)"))
 (segment (start 117.04 63) (end 117.04 66.3) (width 0.2) (layer "F.Cu") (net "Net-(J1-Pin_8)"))
 (segment (start 119.58 66.3) (end 118.88 67) (width 0.2) (layer "F.Cu") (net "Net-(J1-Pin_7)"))
 (segment (start 119.58 63) (end 119.58 66.3) (width 0.2) (layer "F.Cu") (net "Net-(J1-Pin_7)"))
 (segment (start 109 82.5) (end 115.46 76.04) (width 2) (layers "B.Cu" "B.Mask") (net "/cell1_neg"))
 (segment (start 109 85) (end 109 82.5) (width 2) (layers "B.Cu" "B.Mask") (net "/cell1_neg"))
 (segment (start 115.46 76.04) (end 118.5 76.04) (width 2) (layers "B.Cu" "B.Mask") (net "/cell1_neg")))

